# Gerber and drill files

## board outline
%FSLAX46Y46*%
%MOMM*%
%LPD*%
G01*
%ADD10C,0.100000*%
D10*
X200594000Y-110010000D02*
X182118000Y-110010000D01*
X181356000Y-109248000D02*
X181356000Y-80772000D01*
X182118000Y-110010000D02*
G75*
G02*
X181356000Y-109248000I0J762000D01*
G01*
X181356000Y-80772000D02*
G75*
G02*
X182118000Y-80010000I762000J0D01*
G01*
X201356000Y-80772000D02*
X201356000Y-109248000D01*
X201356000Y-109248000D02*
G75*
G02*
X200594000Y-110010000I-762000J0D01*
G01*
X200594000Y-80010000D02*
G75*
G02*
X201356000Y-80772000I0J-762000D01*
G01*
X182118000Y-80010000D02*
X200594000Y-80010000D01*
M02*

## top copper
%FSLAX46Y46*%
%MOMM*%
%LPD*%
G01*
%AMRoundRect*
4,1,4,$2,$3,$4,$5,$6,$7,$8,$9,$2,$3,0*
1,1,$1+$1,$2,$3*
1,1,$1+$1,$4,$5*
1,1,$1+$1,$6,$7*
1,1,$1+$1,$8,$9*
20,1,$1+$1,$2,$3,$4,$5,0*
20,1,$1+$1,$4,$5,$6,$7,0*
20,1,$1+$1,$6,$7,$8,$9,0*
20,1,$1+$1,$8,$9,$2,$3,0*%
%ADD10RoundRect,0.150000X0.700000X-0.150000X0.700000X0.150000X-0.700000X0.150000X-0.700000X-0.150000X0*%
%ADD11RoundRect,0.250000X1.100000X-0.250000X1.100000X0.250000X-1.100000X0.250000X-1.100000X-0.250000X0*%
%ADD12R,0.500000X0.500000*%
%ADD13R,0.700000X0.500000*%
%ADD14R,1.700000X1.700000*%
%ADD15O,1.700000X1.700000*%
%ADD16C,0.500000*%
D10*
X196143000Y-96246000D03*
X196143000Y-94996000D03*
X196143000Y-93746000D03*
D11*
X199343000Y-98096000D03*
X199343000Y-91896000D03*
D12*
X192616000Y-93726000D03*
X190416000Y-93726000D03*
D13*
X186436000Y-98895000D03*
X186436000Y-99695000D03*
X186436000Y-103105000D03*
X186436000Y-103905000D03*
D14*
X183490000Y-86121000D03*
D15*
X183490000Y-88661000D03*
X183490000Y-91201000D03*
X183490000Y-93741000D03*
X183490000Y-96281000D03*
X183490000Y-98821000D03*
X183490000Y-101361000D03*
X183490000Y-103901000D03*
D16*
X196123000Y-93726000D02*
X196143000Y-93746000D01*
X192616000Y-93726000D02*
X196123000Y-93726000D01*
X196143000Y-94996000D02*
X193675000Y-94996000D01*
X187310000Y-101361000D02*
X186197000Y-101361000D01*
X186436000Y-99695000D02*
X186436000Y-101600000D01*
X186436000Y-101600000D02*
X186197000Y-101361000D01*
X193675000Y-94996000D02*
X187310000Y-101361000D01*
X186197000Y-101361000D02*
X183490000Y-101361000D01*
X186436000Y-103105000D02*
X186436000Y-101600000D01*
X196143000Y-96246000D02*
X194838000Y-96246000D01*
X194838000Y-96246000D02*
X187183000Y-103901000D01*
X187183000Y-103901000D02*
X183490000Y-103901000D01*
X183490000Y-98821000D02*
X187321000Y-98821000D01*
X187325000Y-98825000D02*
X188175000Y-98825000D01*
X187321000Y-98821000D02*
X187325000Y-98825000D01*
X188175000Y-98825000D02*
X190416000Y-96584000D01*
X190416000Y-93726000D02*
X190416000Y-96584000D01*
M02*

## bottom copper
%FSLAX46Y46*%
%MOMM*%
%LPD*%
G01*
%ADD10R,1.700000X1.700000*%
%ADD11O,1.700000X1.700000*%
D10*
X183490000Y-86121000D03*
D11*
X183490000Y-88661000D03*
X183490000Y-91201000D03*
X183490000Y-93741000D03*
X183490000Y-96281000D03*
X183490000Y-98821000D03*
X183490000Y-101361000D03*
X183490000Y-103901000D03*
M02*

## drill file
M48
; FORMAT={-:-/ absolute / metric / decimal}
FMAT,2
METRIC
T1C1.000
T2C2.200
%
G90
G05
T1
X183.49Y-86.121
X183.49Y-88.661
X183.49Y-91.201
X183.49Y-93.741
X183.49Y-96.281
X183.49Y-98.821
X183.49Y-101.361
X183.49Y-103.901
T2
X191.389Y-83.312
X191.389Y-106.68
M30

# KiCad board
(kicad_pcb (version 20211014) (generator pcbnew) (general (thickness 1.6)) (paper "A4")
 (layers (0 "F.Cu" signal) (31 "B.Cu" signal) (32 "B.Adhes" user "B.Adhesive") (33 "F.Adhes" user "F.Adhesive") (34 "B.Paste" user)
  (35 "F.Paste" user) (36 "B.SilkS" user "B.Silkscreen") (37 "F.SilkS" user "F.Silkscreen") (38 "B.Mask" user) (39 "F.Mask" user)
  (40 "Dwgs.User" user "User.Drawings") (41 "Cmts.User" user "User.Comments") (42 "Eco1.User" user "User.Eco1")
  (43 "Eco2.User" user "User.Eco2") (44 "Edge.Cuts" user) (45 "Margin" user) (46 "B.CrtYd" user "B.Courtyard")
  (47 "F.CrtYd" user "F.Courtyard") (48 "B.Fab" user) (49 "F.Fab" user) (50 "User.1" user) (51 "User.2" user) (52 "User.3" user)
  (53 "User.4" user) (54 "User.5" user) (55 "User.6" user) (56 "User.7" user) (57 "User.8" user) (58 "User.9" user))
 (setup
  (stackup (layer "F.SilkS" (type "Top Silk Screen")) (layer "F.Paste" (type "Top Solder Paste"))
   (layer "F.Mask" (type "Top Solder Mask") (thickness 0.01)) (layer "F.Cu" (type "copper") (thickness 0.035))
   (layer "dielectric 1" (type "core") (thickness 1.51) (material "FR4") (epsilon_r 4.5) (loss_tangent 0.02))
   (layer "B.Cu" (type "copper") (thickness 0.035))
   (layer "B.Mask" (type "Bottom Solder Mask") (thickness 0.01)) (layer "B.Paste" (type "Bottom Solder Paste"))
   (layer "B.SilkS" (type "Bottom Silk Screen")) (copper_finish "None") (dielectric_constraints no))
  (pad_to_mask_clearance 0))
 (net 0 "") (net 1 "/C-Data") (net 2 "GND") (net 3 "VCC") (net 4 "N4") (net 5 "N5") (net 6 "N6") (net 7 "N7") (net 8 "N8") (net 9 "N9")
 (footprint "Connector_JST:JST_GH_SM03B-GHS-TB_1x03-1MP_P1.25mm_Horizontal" (layer "F.Cu") (at 197.993 94.996 90)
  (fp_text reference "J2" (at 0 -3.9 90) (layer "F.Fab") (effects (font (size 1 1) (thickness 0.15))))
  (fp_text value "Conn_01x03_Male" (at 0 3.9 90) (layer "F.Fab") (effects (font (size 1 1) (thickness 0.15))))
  (pad "1" smd roundrect (at -1.25 -1.85 90) (size 0.6 1.7) (layers "F.Cu" "F.Paste" "F.Mask") (roundrect_rratio 0.25) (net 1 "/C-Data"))
  (pad "2" smd roundrect (at 0 -1.85 90) (size 0.6 1.7) (layers "F.Cu" "F.Paste" "F.Mask") (roundrect_rratio 0.25) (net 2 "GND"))
  (pad "3" smd roundrect (at 1.25 -1.85 90) (size 0.6 1.7) (layers "F.Cu" "F.Paste" "F.Mask") (roundrect_rratio 0.25) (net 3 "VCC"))
  (pad "MP" smd roundrect (at -3.1 1.35 90) (size 1 2.7) (layers "F.Cu" "F.Paste" "F.Mask") (roundrect_rratio 0.25))
  (pad "MP" smd roundrect (at 3.1 1.35 90) (size 1 2.7) (layers "F.Cu" "F.Paste" "F.Mask") (roundrect_rratio 0.25)))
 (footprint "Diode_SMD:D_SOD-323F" (layer "F.Cu") (at 191.516 93.726 180)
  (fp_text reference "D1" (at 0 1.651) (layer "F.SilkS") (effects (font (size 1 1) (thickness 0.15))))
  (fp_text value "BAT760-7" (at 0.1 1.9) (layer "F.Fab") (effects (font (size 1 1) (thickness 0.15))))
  (pad "1" smd rect (at -1.1 0 180) (size 0.5 0.5) (layers "F.Cu" "F.Paste" "F.Mask") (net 3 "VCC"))
  (pad "2" smd rect (at 1.1 0 180) (size 0.5 0.5) (layers "F.Cu" "F.Paste" "F.Mask") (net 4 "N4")))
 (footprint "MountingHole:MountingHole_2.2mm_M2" (layer "F.Cu") (at 191.389 83.312)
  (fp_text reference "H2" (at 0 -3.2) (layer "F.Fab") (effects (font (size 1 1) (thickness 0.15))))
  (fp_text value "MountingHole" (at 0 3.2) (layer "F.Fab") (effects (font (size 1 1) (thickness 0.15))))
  (pad "" np_thru_hole circle (at 0 0) (size 2.2 2.2) (drill 2.2) (layers *.Cu *.Mask)))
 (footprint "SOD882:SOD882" (layer "F.Cu") (at 186.436 99.295 -90) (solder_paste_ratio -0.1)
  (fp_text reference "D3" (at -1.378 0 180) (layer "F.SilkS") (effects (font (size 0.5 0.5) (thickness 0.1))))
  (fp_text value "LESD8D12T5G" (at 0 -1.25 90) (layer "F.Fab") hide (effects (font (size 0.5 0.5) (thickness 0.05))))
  (pad "1" smd rect (at -0.4 0 270) (size 0.5 0.7) (layers "F.Cu" "F.Paste" "F.Mask") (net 4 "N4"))
  (pad "2" smd rect (at 0.4 0 270) (size 0.5 0.7) (layers "F.Cu" "F.Paste" "F.Mask") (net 2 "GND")))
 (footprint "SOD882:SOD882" (layer "F.Cu") (at 186.436 103.505 -90) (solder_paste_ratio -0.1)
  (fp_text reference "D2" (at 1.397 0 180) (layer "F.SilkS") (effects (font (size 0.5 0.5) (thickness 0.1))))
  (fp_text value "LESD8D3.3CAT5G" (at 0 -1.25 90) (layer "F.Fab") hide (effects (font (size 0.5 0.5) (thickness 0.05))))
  (pad "1" smd rect (at -0.4 0 270) (size 0.5 0.7) (layers "F.Cu" "F.Paste" "F.Mask") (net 2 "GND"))
  (pad "2" smd rect (at 0.4 0 270) (size 0.5 0.7) (layers "F.Cu" "F.Paste" "F.Mask") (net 1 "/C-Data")))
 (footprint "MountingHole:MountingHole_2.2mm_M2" (layer "F.Cu") (at 191.389 106.68)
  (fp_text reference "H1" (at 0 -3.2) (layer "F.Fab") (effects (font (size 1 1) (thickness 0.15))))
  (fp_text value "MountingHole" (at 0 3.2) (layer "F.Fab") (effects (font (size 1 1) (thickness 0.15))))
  (pad "" np_thru_hole circle (at 0 0) (size 2.2 2.2) (drill 2.2) (layers *.Cu *.Mask)))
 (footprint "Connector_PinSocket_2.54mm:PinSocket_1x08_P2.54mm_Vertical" (layer "B.Cu") (at 183.49 86.121 180)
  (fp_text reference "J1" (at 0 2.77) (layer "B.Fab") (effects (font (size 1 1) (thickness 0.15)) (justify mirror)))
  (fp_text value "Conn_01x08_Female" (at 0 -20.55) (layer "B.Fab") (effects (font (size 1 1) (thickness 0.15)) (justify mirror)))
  (pad "1" thru_hole rect (at 0 0 180) (size 1.7 1.7) (drill 1) (layers *.Cu *.Mask) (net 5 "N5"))
  (pad "2" thru_hole oval (at 0 -2.54 180) (size 1.7 1.7) (drill 1) (layers *.Cu *.Mask) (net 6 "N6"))
  (pad "3" thru_hole oval (at 0 -5.08 180) (size 1.7 1.7) (drill 1) (layers *.Cu *.Mask) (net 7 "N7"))
  (pad "4" thru_hole oval (at 0 -7.62 180) (size 1.7 1.7) (drill 1) (layers *.Cu *.Mask) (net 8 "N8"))
  (pad "5" thru_hole oval (at 0 -10.16 180) (size 1.7 1.7) (drill 1) (layers *.Cu *.Mask) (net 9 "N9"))
  (pad "6" thru_hole oval (at 0 -12.7 180) (size 1.7 1.7) (drill 1) (layers *.Cu *.Mask) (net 4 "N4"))
  (pad "7" thru_hole oval (at 0 -15.24 180) (size 1.7 1.7) (drill 1) (layers *.Cu *.Mask) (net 2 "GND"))
  (pad "8" thru_hole oval (at 0 -17.78 180) (size 1.7 1.7) (drill 1) (layers *.Cu *.Mask) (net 1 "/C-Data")))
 (gr_line (start 200.594 110.01) (end 182.118 110.01) (layer "Edge.Cuts") (width 0.1))
 (gr_line (start 181.356 109.248) (end 181.356 80.772) (layer "Edge.Cuts") (width 0.1))
 (gr_arc (start 182.118 110.01) (mid 181.579185 109.786815) (end 181.356 109.248) (layer "Edge.Cuts") (width 0.1))
 (gr_arc (start 181.356 80.772) (mid 181.579185 80.233185) (end 182.118 80.01) (layer "Edge.Cuts") (width 0.1))
 (gr_line (start 201.356 80.772) (end 201.356 109.248) (layer "Edge.Cuts") (width 0.1))
 (gr_arc (start 201.356 109.248) (mid 201.132815 109.786815) (end 200.594 110.01) (layer "Edge.Cuts") (width 0.1))
 (gr_arc (start 200.594 80.01) (mid 201.132815 80.233185) (end 201.356 80.772) (layer "Edge.Cuts") (width 0.1))
 (gr_line (start 182.118 80.01) (end 200.594 80.01) (layer "Edge.Cuts") (width 0.1))
 (segment (start 196.123 93.726) (end 196.143 93.746) (width 0.5) (layer "F.Cu") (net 3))
 (segment (start 192.616 93.726) (end 196.123 93.726) (width 0.5) (layer "F.Cu") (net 3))
 (segment (start 196.143 94.996) (end 193.675 94.996) (width 0.5) (layer "F.Cu") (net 2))
 (segment (start 187.31 101.361) (end 186.197 101.361) (width 0.5) (layer "F.Cu") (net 2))
 (segment (start 186.436 99.695) (end 186.436 101.6) (width 0.5) (layer "F.Cu") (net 2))
 (segment (start 186.436 101.6) (end 186.197 101.361) (width 0.5) (layer "F.Cu") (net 2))
 (segment (start 193.675 94.996) (end 187.31 101.361) (width 0.5) (layer "F.Cu") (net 2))
 (segment (start 186.197 101.361) (end 183.49 101.361) (width 0.5) (layer "F.Cu") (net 2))
 (segment (start 186.436 103.105) (end 186.436 101.6) (width 0.5) (layer "F.Cu") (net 2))
 (segment (start 196.143 96.246) (end 194.838 96.246) (width 0.5) (layer "F.Cu") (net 1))
 (segment (start 194.838 96.246) (end 187.183 103.901) (width 0.5) (layer "F.Cu") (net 1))
 (segment (start 187.183 103.901) (end 183.49 103.901) (width 0.5) (layer "F.Cu") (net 1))
 (segment (start 183.49 98.821) (end 187.321 98.821) (width 0.5) (layer "F.Cu") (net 4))
 (segment (start 187.325 98.825) (end 188.175 98.825) (width 0.5) (layer "F.Cu") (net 4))
 (segment (start 187.321 98.821) (end 187.325 98.825) (width 0.5) (layer "F.Cu") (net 4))
 (segment (start 188.175 98.825) (end 190.416 96.584) (width 0.5) (layer "F.Cu") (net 4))
 (segment (start 190.416 93.726) (end 190.416 96.584) (width 0.5) (layer "F.Cu") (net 4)))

